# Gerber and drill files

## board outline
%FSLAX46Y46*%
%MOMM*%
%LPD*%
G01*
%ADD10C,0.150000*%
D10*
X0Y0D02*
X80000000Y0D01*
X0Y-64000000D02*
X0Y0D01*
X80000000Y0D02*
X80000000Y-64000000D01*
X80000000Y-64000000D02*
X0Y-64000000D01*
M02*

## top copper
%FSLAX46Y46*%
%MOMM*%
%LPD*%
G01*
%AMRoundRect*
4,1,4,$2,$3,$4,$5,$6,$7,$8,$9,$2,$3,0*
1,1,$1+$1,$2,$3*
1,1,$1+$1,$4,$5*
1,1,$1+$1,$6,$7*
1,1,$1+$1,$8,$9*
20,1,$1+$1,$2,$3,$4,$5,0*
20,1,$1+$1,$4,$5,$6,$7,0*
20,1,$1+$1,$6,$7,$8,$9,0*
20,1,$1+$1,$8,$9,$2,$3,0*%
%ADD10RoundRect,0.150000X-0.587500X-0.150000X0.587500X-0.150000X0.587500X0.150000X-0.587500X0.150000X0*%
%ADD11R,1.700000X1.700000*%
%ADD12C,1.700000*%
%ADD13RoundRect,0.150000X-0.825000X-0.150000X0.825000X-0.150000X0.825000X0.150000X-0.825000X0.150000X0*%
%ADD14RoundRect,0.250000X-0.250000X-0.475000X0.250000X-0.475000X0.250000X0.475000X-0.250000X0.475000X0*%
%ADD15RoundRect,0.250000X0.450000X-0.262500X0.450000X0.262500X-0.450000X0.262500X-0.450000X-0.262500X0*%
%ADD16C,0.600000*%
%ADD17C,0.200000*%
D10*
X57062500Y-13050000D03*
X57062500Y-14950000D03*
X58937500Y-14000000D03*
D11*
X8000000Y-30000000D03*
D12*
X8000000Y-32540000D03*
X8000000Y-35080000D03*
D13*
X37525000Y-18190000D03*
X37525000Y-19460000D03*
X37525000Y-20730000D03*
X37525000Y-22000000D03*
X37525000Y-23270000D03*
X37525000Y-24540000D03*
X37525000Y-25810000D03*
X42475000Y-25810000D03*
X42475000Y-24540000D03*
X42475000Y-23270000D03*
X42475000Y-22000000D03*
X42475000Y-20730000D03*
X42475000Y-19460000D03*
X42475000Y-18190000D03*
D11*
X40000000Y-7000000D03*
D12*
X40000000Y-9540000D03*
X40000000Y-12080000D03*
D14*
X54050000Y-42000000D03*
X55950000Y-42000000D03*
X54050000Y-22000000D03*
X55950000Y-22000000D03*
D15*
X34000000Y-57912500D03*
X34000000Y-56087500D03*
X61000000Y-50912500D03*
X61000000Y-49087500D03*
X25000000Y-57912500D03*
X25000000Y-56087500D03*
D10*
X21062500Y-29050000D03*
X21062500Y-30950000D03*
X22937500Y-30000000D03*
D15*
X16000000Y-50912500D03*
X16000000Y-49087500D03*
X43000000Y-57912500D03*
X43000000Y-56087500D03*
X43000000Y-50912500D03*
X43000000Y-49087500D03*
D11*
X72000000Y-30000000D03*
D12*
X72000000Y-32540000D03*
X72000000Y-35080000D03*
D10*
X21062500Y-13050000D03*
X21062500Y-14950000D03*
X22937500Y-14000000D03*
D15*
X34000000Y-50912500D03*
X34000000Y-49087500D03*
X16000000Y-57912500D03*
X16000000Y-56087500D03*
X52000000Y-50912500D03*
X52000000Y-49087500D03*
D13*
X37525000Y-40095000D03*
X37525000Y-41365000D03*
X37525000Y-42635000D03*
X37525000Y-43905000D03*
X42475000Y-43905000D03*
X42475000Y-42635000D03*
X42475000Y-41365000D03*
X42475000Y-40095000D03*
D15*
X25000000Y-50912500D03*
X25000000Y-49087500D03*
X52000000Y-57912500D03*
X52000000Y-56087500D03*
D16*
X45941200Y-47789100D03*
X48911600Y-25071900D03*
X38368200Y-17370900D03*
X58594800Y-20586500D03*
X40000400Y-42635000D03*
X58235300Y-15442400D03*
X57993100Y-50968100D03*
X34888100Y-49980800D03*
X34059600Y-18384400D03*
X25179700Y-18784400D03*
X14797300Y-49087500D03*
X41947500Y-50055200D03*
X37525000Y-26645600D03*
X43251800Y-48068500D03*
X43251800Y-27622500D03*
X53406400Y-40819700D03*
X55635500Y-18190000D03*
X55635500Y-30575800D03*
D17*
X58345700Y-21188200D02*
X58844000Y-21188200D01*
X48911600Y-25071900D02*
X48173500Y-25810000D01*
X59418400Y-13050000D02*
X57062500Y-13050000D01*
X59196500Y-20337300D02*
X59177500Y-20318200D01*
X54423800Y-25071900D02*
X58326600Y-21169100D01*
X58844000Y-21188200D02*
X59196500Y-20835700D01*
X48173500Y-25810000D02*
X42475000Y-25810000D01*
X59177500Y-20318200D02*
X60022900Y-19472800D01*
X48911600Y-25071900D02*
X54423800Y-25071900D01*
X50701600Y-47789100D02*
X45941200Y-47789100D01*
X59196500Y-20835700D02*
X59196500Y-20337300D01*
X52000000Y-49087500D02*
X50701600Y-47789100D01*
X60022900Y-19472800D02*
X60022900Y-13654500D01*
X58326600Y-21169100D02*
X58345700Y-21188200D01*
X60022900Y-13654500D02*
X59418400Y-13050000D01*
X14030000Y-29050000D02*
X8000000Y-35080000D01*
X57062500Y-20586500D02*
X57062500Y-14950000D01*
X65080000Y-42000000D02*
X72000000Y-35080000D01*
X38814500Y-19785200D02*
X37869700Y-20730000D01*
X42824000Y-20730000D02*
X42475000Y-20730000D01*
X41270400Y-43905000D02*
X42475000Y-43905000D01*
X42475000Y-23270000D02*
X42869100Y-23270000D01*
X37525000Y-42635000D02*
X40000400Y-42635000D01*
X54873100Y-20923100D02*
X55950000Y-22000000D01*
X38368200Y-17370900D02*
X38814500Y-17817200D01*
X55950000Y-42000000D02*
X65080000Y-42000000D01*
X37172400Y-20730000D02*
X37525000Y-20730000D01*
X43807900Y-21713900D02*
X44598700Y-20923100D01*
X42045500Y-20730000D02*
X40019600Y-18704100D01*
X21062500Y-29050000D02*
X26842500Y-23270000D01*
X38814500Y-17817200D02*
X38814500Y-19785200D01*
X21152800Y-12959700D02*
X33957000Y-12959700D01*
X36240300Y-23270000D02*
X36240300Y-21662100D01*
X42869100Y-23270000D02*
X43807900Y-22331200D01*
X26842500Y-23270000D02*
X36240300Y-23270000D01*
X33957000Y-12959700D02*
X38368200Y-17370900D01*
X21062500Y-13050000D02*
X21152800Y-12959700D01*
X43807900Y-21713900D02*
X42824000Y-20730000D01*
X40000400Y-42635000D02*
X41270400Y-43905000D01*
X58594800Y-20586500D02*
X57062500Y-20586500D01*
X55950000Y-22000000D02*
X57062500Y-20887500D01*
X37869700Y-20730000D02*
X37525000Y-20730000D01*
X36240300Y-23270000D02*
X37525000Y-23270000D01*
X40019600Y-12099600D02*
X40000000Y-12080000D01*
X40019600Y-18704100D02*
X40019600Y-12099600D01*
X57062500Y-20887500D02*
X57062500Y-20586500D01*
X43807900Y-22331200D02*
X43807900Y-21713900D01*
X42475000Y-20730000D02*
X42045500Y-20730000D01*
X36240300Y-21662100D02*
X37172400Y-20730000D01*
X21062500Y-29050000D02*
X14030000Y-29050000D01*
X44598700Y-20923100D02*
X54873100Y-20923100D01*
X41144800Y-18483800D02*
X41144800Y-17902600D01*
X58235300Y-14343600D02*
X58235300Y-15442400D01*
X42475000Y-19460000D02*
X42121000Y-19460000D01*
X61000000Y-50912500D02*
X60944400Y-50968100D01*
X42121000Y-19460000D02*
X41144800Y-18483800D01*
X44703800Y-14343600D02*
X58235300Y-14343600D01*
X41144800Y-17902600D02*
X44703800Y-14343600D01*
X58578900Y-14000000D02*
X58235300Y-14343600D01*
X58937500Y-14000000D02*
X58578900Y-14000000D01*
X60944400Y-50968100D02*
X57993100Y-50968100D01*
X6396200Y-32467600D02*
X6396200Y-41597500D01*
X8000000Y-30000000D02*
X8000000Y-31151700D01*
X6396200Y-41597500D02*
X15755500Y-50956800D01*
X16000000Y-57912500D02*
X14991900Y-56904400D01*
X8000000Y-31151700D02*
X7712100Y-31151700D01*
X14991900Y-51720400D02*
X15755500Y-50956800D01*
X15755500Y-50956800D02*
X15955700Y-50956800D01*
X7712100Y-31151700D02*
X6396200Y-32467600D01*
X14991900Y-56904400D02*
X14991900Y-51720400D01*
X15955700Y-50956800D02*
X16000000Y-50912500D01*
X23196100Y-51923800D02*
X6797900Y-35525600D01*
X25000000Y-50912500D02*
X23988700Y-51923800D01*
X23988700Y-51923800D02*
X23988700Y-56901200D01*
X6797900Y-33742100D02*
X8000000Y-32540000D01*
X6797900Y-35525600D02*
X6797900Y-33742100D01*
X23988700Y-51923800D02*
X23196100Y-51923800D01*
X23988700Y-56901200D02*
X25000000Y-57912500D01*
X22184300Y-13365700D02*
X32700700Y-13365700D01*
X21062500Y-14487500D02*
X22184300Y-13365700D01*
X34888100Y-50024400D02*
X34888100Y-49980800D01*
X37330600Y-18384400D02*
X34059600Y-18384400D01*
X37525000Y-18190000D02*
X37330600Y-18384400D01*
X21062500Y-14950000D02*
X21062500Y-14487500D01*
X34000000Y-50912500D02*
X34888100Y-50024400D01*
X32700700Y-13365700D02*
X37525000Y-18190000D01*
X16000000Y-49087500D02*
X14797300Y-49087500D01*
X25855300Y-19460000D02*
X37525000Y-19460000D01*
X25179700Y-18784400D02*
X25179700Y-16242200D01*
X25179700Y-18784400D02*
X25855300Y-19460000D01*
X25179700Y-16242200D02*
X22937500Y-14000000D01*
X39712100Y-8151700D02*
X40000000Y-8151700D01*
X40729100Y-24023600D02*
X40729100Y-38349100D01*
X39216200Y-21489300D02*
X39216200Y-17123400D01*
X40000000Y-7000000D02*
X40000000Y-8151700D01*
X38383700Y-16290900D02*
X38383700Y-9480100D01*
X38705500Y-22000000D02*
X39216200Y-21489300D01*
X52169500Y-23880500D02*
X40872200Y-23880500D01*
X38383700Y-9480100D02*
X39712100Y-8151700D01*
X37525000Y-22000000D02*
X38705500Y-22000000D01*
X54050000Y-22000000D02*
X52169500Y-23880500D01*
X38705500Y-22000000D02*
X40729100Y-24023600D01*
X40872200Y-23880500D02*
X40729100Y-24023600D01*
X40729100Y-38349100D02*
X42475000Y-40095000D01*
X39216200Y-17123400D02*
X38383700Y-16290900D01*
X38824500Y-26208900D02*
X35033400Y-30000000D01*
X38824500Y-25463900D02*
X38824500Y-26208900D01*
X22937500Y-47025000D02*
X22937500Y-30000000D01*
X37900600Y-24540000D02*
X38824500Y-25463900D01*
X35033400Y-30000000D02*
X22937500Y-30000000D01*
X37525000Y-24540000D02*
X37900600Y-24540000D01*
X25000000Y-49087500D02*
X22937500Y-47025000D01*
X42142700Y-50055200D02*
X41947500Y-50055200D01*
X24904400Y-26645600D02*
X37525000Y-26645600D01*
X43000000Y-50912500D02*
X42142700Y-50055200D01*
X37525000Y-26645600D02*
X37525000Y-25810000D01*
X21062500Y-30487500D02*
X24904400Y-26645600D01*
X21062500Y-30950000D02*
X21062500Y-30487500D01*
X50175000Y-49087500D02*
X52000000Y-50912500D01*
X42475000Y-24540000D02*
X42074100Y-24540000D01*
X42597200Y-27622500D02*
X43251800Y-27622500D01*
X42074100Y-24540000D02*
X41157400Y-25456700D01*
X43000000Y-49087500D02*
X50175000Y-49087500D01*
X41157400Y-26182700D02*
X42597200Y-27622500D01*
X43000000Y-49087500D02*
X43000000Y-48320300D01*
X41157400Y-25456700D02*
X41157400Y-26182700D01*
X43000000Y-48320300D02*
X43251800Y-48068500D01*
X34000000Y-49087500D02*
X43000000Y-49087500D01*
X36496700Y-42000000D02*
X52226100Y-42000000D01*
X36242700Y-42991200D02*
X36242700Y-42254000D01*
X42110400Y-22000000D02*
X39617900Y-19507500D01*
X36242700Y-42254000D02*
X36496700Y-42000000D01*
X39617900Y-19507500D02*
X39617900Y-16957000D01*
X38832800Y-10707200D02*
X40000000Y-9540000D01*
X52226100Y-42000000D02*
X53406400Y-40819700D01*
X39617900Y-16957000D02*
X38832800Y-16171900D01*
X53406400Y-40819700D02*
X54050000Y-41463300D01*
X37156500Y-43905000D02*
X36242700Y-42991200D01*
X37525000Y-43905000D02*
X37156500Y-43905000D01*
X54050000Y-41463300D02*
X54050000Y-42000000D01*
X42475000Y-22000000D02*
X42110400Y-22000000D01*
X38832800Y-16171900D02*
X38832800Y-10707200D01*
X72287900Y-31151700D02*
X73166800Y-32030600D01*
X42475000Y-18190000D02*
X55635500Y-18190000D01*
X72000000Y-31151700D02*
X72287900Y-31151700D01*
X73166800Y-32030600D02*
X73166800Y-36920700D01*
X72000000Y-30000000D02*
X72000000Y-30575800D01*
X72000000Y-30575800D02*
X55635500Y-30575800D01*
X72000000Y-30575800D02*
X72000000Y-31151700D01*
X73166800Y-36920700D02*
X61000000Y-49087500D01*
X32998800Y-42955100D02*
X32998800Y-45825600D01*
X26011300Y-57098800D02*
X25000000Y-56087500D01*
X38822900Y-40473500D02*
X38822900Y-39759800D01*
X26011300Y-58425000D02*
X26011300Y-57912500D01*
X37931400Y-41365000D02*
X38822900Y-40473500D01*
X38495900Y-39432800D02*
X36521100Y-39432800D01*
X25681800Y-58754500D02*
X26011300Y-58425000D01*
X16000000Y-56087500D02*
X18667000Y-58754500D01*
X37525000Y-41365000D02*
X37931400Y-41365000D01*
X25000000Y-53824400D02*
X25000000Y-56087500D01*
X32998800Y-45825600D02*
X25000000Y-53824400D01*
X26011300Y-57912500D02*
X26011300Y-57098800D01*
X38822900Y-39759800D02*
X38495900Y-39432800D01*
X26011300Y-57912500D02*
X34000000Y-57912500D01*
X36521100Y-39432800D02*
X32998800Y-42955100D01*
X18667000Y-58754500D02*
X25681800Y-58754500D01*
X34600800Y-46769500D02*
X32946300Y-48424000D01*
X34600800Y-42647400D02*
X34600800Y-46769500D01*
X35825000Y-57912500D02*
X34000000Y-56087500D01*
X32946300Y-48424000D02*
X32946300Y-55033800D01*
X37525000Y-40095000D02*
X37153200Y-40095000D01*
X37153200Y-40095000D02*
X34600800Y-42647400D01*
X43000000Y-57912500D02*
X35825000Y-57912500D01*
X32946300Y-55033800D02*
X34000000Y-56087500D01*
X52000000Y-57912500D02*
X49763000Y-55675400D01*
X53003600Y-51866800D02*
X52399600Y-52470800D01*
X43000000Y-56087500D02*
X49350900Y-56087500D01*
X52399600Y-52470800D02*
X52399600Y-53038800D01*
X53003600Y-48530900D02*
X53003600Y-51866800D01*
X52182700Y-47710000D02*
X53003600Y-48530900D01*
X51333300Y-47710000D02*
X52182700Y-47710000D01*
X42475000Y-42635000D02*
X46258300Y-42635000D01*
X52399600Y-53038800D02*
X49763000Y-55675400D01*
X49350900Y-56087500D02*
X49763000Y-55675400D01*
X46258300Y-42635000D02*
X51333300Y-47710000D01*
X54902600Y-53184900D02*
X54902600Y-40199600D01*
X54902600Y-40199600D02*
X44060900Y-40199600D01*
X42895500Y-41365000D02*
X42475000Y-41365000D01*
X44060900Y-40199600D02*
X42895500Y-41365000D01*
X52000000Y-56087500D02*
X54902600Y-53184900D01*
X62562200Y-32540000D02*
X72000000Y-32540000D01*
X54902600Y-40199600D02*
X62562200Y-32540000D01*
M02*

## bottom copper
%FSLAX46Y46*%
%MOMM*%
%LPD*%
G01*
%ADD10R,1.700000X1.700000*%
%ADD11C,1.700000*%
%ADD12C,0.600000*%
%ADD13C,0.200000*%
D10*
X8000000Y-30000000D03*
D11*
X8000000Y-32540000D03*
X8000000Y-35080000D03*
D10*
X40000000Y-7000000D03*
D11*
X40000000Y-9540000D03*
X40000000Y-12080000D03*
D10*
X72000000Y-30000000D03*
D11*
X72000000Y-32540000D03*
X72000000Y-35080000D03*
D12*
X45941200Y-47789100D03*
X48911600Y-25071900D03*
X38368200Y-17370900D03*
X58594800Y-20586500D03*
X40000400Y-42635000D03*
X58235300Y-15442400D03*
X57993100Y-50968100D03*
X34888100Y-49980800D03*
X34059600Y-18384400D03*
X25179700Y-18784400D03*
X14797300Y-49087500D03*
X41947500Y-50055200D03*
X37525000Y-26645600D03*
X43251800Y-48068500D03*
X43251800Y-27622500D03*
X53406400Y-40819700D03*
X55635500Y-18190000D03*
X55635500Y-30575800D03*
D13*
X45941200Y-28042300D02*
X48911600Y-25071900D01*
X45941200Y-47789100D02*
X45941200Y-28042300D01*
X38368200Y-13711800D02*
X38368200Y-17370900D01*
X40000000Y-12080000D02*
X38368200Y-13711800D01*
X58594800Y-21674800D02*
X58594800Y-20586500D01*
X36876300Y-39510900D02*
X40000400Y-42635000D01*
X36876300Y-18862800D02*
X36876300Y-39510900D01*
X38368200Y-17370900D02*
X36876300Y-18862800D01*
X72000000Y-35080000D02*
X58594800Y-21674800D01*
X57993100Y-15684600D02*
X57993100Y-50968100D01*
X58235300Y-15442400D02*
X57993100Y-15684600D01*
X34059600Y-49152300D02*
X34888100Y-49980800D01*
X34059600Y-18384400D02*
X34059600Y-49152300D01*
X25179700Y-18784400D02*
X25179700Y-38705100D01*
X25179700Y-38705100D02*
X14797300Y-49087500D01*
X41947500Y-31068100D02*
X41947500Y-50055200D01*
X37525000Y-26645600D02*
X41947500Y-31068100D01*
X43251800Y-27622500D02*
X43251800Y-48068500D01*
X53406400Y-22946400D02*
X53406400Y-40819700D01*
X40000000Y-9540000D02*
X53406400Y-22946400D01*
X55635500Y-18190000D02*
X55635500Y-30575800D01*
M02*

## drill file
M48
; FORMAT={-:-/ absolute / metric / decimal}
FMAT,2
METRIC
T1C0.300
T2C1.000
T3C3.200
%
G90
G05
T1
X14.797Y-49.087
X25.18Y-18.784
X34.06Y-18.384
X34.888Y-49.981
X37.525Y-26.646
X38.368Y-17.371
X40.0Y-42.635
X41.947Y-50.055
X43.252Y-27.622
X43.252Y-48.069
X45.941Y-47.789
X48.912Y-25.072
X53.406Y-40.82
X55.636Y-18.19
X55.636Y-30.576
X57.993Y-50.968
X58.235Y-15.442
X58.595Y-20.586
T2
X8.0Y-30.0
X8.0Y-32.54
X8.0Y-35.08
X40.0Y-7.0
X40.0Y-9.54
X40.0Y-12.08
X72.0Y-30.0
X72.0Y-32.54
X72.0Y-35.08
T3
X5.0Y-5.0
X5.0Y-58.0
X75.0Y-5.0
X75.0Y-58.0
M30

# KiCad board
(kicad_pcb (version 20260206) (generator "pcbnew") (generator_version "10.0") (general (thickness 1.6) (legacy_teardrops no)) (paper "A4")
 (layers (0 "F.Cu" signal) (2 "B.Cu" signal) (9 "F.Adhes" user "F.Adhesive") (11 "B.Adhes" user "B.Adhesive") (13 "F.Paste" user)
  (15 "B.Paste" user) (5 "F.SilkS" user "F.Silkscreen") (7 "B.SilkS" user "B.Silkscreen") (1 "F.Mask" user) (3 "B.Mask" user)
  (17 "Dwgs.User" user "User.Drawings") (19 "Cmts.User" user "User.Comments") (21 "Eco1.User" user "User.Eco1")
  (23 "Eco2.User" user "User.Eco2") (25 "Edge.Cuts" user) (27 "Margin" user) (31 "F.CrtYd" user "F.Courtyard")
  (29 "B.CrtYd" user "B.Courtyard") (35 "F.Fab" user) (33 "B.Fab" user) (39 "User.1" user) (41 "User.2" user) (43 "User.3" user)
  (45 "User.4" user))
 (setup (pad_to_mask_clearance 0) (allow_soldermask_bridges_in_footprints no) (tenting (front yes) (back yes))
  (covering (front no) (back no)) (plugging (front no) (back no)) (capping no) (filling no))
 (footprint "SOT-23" (layer "F.Cu") (at 58 14)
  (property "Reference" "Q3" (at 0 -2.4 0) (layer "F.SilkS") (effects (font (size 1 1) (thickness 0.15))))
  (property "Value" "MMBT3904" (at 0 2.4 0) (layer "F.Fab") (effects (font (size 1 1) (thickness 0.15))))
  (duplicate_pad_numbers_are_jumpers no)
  (pad "1" smd roundrect (at -0.9375 -0.95) (size 1.475 0.6) (layers "F.Cu" "F.Mask" "F.Paste") (roundrect_rratio 0.25) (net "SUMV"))
  (pad "2" smd roundrect (at -0.9375 0.95) (size 1.475 0.6) (layers "F.Cu" "F.Mask" "F.Paste") (roundrect_rratio 0.25) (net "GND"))
  (pad "3" smd roundrect (at 0.9375 0) (size 1.475 0.6) (layers "F.Cu" "F.Mask" "F.Paste") (roundrect_rratio 0.25) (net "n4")))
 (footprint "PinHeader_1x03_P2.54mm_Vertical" (layer "F.Cu") (at 8 30)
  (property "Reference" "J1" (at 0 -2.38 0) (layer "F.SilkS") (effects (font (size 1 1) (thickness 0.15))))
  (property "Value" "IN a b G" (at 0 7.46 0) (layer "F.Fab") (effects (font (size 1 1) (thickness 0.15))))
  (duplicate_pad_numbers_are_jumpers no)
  (pad "1" thru_hole rect (at 0 0) (size 1.7 1.7) (drill 1) (layers "*.Cu" "*.Mask") (remove_unused_layers no) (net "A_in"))
  (pad "2" thru_hole circle (at 0 2.54) (size 1.7 1.7) (drill 1) (layers "*.Cu" "*.Mask") (remove_unused_layers no) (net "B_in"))
  (pad "3" thru_hole circle (at 0 5.08) (size 1.7 1.7) (drill 1) (layers "*.Cu" "*.Mask") (remove_unused_layers no) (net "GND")))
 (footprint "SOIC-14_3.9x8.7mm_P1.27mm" (layer "F.Cu") (at 40 22)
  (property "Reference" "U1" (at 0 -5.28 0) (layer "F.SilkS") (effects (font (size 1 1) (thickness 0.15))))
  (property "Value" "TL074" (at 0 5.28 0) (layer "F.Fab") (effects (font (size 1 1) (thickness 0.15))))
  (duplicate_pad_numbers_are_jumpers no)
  (pad "1" smd roundrect (at -2.475 -3.81) (size 1.95 0.6) (layers "F.Cu" "F.Mask" "F.Paste") (roundrect_rratio 0.25) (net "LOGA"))
  (pad "2" smd roundrect (at -2.475 -2.54) (size 1.95 0.6) (layers "F.Cu" "F.Mask" "F.Paste") (roundrect_rratio 0.25) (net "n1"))
  (pad "3" smd roundrect (at -2.475 -1.27) (size 1.95 0.6) (layers "F.Cu" "F.Mask" "F.Paste") (roundrect_rratio 0.25) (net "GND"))
  (pad "4" smd roundrect (at -2.475 0) (size 1.95 0.6) (layers "F.Cu" "F.Mask" "F.Paste") (roundrect_rratio 0.25) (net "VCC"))
  (pad "5" smd roundrect (at -2.475 1.27) (size 1.95 0.6) (layers "F.Cu" "F.Mask" "F.Paste") (roundrect_rratio 0.25) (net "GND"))
  (pad "6" smd roundrect (at -2.475 2.54) (size 1.95 0.6) (layers "F.Cu" "F.Mask" "F.Paste") (roundrect_rratio 0.25) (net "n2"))
  (pad "7" smd roundrect (at -2.475 3.81) (size 1.95 0.6) (layers "F.Cu" "F.Mask" "F.Paste") (roundrect_rratio 0.25) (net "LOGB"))
  (pad "8" smd roundrect (at 2.475 3.81) (size 1.95 0.6) (layers "F.Cu" "F.Mask" "F.Paste") (roundrect_rratio 0.25) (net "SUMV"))
  (pad "9" smd roundrect (at 2.475 2.54) (size 1.95 0.6) (layers "F.Cu" "F.Mask" "F.Paste") (roundrect_rratio 0.25) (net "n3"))
  (pad "10" smd roundrect (at 2.475 1.27) (size 1.95 0.6) (layers "F.Cu" "F.Mask" "F.Paste") (roundrect_rratio 0.25) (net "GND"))
  (pad "11" smd roundrect (at 2.475 0) (size 1.95 0.6) (layers "F.Cu" "F.Mask" "F.Paste") (roundrect_rratio 0.25) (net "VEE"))
  (pad "12" smd roundrect (at 2.475 -1.27) (size 1.95 0.6) (layers "F.Cu" "F.Mask" "F.Paste") (roundrect_rratio 0.25) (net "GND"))
  (pad "13" smd roundrect (at 2.475 -2.54) (size 1.95 0.6) (layers "F.Cu" "F.Mask" "F.Paste") (roundrect_rratio 0.25) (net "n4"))
  (pad "14" smd roundrect (at 2.475 -3.81) (size 1.95 0.6) (layers "F.Cu" "F.Mask" "F.Paste") (roundrect_rratio 0.25) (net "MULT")))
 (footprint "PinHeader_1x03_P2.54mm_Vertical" (layer "F.Cu") (at 40 7)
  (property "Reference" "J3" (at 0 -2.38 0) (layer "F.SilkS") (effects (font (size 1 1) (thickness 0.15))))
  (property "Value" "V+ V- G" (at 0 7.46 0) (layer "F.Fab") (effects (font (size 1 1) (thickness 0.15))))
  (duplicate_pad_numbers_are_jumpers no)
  (pad "1" thru_hole rect (at 0 0) (size 1.7 1.7) (drill 1) (layers "*.Cu" "*.Mask") (remove_unused_layers no) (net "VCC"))
  (pad "2" thru_hole circle (at 0 2.54) (size 1.7 1.7) (drill 1) (layers "*.Cu" "*.Mask") (remove_unused_layers no) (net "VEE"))
  (pad "3" thru_hole circle (at 0 5.08) (size 1.7 1.7) (drill 1) (layers "*.Cu" "*.Mask") (remove_unused_layers no) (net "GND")))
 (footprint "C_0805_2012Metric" (layer "F.Cu") (at 55 42)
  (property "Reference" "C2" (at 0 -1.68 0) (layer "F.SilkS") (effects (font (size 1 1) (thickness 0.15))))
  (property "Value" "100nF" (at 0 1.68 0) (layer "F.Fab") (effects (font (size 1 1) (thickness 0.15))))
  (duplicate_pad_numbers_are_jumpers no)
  (pad "1" smd roundrect (at -0.95 0) (size 1 1.45) (layers "F.Cu" "F.Mask" "F.Paste") (roundrect_rratio 0.25) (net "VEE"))
  (pad "2" smd roundrect (at 0.95 0) (size 1 1.45) (layers "F.Cu" "F.Mask" "F.Paste") (roundrect_rratio 0.25) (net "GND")))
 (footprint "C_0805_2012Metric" (layer "F.Cu") (at 55 22)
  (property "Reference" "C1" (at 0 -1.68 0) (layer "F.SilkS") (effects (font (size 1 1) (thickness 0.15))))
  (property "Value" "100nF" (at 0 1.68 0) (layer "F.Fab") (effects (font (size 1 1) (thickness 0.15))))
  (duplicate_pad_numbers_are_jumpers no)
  (pad "1" smd roundrect (at -0.95 0) (size 1 1.45) (layers "F.Cu" "F.Mask" "F.Paste") (roundrect_rratio 0.25) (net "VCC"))
  (pad "2" smd roundrect (at 0.95 0) (size 1 1.45) (layers "F.Cu" "F.Mask" "F.Paste") (roundrect_rratio 0.25) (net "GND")))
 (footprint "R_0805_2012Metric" (layer "F.Cu") (at 34 57 90)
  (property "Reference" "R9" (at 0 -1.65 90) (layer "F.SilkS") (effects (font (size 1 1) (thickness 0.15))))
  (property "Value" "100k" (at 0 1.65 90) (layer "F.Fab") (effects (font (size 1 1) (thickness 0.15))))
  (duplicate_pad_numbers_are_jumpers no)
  (pad "1" smd roundrect (at -0.9125 0 90) (size 1.025 1.4) (layers "F.Cu" "F.Mask" "F.Paste") (roundrect_rratio 0.243902) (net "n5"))
  (pad "2" smd roundrect (at 0.9125 0 90) (size 1.025 1.4) (layers "F.Cu" "F.Mask" "F.Paste") (roundrect_rratio 0.243902) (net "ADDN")))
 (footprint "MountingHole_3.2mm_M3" (layer "F.Cu") (at 5 58)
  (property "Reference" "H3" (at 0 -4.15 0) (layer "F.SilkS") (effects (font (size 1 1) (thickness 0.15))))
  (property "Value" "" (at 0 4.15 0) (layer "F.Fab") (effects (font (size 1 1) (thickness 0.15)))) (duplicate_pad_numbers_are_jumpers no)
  (pad "" np_thru_hole circle (at 0 0) (size 3.2 3.2) (drill 3.2) (layers "*.Cu" "*.Mask")))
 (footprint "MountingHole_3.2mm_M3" (layer "F.Cu") (at 75 5)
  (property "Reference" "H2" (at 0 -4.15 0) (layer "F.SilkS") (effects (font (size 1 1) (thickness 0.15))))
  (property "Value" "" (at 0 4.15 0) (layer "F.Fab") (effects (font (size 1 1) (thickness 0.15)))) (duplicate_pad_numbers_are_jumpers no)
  (pad "" np_thru_hole circle (at 0 0) (size 3.2 3.2) (drill 3.2) (layers "*.Cu" "*.Mask")))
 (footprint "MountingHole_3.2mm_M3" (layer "F.Cu") (at 5 5)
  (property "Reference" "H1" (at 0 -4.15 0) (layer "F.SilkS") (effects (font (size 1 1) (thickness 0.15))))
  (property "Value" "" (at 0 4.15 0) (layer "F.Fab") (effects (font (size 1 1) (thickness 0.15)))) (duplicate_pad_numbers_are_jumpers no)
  (pad "" np_thru_hole circle (at 0 0) (size 3.2 3.2) (drill 3.2) (layers "*.Cu" "*.Mask")))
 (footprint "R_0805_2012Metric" (layer "F.Cu") (at 61 50 90)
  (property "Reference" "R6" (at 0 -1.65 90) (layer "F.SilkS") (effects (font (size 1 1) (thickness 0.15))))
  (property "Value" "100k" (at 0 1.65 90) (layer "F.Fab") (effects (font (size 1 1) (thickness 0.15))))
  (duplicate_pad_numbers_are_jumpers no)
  (pad "1" smd roundrect (at -0.9125 0 90) (size 1.025 1.4) (layers "F.Cu" "F.Mask" "F.Paste") (roundrect_rratio 0.243902) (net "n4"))
  (pad "2" smd roundrect (at 0.9125 0 90) (size 1.025 1.4) (layers "F.Cu" "F.Mask" "F.Paste") (roundrect_rratio 0.243902) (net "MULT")))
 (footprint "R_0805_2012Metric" (layer "F.Cu") (at 25 57 90)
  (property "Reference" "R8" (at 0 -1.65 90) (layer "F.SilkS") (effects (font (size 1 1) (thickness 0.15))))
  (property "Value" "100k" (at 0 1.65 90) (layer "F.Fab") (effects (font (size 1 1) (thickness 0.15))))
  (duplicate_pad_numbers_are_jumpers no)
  (pad "1" smd roundrect (at -0.9125 0 90) (size 1.025 1.4) (layers "F.Cu" "F.Mask" "F.Paste") (roundrect_rratio 0.243902) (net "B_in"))
  (pad "2" smd roundrect (at 0.9125 0 90) (size 1.025 1.4) (layers "F.Cu" "F.Mask" "F.Paste") (roundrect_rratio 0.243902) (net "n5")))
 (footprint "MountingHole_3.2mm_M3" (layer "F.Cu") (at 75 58)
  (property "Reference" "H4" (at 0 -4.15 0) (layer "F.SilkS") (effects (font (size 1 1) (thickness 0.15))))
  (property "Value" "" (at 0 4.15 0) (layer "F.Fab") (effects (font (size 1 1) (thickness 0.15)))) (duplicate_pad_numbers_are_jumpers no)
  (pad "" np_thru_hole circle (at 0 0) (size 3.2 3.2) (drill 3.2) (layers "*.Cu" "*.Mask")))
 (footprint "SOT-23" (layer "F.Cu") (at 22 30)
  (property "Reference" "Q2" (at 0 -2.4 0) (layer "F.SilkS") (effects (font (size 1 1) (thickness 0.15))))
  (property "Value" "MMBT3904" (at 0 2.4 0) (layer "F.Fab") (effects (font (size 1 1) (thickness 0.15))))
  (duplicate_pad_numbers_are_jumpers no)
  (pad "1" smd roundrect (at -0.9375 -0.95) (size 1.475 0.6) (layers "F.Cu" "F.Mask" "F.Paste") (roundrect_rratio 0.25) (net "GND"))
  (pad "2" smd roundrect (at -0.9375 0.95) (size 1.475 0.6) (layers "F.Cu" "F.Mask" "F.Paste") (roundrect_rratio 0.25) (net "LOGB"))
  (pad "3" smd roundrect (at 0.9375 0) (size 1.475 0.6) (layers "F.Cu" "F.Mask" "F.Paste") (roundrect_rratio 0.25) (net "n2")))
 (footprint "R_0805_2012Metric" (layer "F.Cu") (at 16 50 90)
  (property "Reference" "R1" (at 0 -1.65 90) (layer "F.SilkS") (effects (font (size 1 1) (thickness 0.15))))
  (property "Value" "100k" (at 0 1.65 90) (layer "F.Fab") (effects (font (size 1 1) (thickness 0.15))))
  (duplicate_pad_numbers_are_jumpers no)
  (pad "1" smd roundrect (at -0.9125 0 90) (size 1.025 1.4) (layers "F.Cu" "F.Mask" "F.Paste") (roundrect_rratio 0.243902) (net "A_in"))
  (pad "2" smd roundrect (at 0.9125 0 90) (size 1.025 1.4) (layers "F.Cu" "F.Mask" "F.Paste") (roundrect_rratio 0.243902) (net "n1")))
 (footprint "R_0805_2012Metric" (layer "F.Cu") (at 43 57 90)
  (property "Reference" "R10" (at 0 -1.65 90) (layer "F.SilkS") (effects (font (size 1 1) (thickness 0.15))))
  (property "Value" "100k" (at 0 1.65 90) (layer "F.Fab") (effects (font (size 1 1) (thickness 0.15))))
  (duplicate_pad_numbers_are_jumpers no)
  (pad "1" smd roundrect (at -0.9125 0 90) (size 1.025 1.4) (layers "F.Cu" "F.Mask" "F.Paste") (roundrect_rratio 0.243902) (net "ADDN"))
  (pad "2" smd roundrect (at 0.9125 0 90) (size 1.025 1.4) (layers "F.Cu" "F.Mask" "F.Paste") (roundrect_rratio 0.243902) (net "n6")))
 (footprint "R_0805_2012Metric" (layer "F.Cu") (at 43 50 90)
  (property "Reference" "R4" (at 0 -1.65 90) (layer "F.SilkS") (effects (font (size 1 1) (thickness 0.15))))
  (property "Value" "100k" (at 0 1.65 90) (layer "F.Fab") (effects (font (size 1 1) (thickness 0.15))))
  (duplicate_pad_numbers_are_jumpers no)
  (pad "1" smd roundrect (at -0.9125 0 90) (size 1.025 1.4) (layers "F.Cu" "F.Mask" "F.Paste") (roundrect_rratio 0.243902) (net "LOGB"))
  (pad "2" smd roundrect (at 0.9125 0 90) (size 1.025 1.4) (layers "F.Cu" "F.Mask" "F.Paste") (roundrect_rratio 0.243902) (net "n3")))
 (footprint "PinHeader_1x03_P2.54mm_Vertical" (layer "F.Cu") (at 72 30)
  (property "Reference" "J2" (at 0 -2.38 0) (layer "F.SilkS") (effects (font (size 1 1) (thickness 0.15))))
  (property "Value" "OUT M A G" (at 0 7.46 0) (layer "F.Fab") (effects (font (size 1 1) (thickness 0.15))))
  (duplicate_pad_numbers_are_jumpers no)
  (pad "1" thru_hole rect (at 0 0) (size 1.7 1.7) (drill 1) (layers "*.Cu" "*.Mask") (remove_unused_layers no) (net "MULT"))
  (pad "2" thru_hole circle (at 0 2.54) (size 1.7 1.7) (drill 1) (layers "*.Cu" "*.Mask") (remove_unused_layers no) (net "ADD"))
  (pad "3" thru_hole circle (at 0 5.08) (size 1.7 1.7) (drill 1) (layers "*.Cu" "*.Mask") (remove_unused_layers no) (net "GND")))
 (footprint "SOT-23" (layer "F.Cu") (at 22 14)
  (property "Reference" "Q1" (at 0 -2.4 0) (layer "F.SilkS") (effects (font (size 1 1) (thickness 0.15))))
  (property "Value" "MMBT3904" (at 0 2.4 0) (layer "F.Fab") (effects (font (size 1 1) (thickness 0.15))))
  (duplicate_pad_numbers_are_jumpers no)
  (pad "1" smd roundrect (at -0.9375 -0.95) (size 1.475 0.6) (layers "F.Cu" "F.Mask" "F.Paste") (roundrect_rratio 0.25) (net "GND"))
  (pad "2" smd roundrect (at -0.9375 0.95) (size 1.475 0.6) (layers "F.Cu" "F.Mask" "F.Paste") (roundrect_rratio 0.25) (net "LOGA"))
  (pad "3" smd roundrect (at 0.9375 0) (size 1.475 0.6) (layers "F.Cu" "F.Mask" "F.Paste") (roundrect_rratio 0.25) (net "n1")))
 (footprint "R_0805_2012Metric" (layer "F.Cu") (at 34 50 90)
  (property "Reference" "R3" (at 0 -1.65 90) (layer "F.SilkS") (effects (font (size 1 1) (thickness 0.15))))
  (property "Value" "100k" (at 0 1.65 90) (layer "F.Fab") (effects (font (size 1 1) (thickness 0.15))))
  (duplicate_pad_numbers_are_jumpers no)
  (pad "1" smd roundrect (at -0.9125 0 90) (size 1.025 1.4) (layers "F.Cu" "F.Mask" "F.Paste") (roundrect_rratio 0.243902) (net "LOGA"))
  (pad "2" smd roundrect (at 0.9125 0 90) (size 1.025 1.4) (layers "F.Cu" "F.Mask" "F.Paste") (roundrect_rratio 0.243902) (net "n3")))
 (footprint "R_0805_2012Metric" (layer "F.Cu") (at 16 57 90)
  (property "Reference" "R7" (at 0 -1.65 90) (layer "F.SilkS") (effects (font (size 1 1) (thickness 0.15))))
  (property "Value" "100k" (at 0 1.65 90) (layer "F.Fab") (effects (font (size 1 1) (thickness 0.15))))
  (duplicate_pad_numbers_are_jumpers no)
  (pad "1" smd roundrect (at -0.9125 0 90) (size 1.025 1.4) (layers "F.Cu" "F.Mask" "F.Paste") (roundrect_rratio 0.243902) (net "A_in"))
  (pad "2" smd roundrect (at 0.9125 0 90) (size 1.025 1.4) (layers "F.Cu" "F.Mask" "F.Paste") (roundrect_rratio 0.243902) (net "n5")))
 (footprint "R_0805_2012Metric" (layer "F.Cu") (at 52 50 90)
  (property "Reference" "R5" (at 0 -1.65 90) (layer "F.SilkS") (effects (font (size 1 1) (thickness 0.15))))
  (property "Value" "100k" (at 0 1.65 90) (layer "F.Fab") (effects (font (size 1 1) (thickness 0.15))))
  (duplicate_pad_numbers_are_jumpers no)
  (pad "1" smd roundrect (at -0.9125 0 90) (size 1.025 1.4) (layers "F.Cu" "F.Mask" "F.Paste") (roundrect_rratio 0.243902) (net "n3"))
  (pad "2" smd roundrect (at 0.9125 0 90) (size 1.025 1.4) (layers "F.Cu" "F.Mask" "F.Paste") (roundrect_rratio 0.243902) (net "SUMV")))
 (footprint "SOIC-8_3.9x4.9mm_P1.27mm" (layer "F.Cu") (at 40 42)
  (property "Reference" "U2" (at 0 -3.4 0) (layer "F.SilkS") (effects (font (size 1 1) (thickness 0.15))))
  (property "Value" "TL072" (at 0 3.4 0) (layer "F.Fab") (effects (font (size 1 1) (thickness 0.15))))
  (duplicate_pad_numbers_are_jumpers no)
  (pad "1" smd roundrect (at -2.475 -1.905) (size 1.95 0.6) (layers "F.Cu" "F.Mask" "F.Paste") (roundrect_rratio 0.25) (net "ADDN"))
  (pad "2" smd roundrect (at -2.475 -0.635) (size 1.95 0.6) (layers "F.Cu" "F.Mask" "F.Paste") (roundrect_rratio 0.25) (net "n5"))
  (pad "3" smd roundrect (at -2.475 0.635) (size 1.95 0.6) (layers "F.Cu" "F.Mask" "F.Paste") (roundrect_rratio 0.25) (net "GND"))
  (pad "4" smd roundrect (at -2.475 1.905) (size 1.95 0.6) (layers "F.Cu" "F.Mask" "F.Paste") (roundrect_rratio 0.25) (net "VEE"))
  (pad "5" smd roundrect (at 2.475 1.905) (size 1.95 0.6) (layers "F.Cu" "F.Mask" "F.Paste") (roundrect_rratio 0.25) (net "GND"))
  (pad "6" smd roundrect (at 2.475 0.635) (size 1.95 0.6) (layers "F.Cu" "F.Mask" "F.Paste") (roundrect_rratio 0.25) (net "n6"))
  (pad "7" smd roundrect (at 2.475 -0.635) (size 1.95 0.6) (layers "F.Cu" "F.Mask" "F.Paste") (roundrect_rratio 0.25) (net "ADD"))
  (pad "8" smd roundrect (at 2.475 -1.905) (size 1.95 0.6) (layers "F.Cu" "F.Mask" "F.Paste") (roundrect_rratio 0.25) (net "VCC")))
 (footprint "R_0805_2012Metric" (layer "F.Cu") (at 25 50 90)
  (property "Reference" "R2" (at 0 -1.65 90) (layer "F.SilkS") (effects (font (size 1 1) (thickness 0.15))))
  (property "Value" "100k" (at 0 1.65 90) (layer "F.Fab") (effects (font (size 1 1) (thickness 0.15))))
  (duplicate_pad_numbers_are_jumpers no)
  (pad "1" smd roundrect (at -0.9125 0 90) (size 1.025 1.4) (layers "F.Cu" "F.Mask" "F.Paste") (roundrect_rratio 0.243902) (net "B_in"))
  (pad "2" smd roundrect (at 0.9125 0 90) (size 1.025 1.4) (layers "F.Cu" "F.Mask" "F.Paste") (roundrect_rratio 0.243902) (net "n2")))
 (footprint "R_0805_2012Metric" (layer "F.Cu") (at 52 57 90)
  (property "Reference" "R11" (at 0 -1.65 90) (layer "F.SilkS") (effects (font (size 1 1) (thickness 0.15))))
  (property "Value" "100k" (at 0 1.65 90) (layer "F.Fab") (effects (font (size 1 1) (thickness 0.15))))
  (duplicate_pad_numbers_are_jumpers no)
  (pad "1" smd roundrect (at -0.9125 0 90) (size 1.025 1.4) (layers "F.Cu" "F.Mask" "F.Paste") (roundrect_rratio 0.243902) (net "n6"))
  (pad "2" smd roundrect (at 0.9125 0 90) (size 1.025 1.4) (layers "F.Cu" "F.Mask" "F.Paste") (roundrect_rratio 0.243902) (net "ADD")))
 (gr_line (start 0 0) (end 80 0) (stroke (width 0.15) (type default)) (layer "Edge.Cuts"))
 (gr_line (start 0 64) (end 0 0) (stroke (width 0.15) (type default)) (layer "Edge.Cuts"))
 (gr_line (start 80 0) (end 80 64) (stroke (width 0.15) (type default)) (layer "Edge.Cuts"))
 (gr_line (start 80 64) (end 0 64) (stroke (width 0.15) (type default)) (layer "Edge.Cuts"))
 (segment (start 58.3457 21.1882) (end 58.844 21.1882) (width 0.2) (layer "F.Cu") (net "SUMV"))
 (segment (start 48.9116 25.0719) (end 48.1735 25.81) (width 0.2) (layer "F.Cu") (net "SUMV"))
 (segment (start 59.4184 13.05) (end 57.0625 13.05) (width 0.2) (layer "F.Cu") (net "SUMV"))
 (segment (start 59.1965 20.3373) (end 59.1775 20.3182) (width 0.2) (layer "F.Cu") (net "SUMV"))
 (segment (start 54.4238 25.0719) (end 58.3266 21.1691) (width 0.2) (layer "F.Cu") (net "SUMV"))
 (segment (start 58.844 21.1882) (end 59.1965 20.8357) (width 0.2) (layer "F.Cu") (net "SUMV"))
 (segment (start 48.1735 25.81) (end 42.475 25.81) (width 0.2) (layer "F.Cu") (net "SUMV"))
 (segment (start 59.1775 20.3182) (end 60.0229 19.4728) (width 0.2) (layer "F.Cu") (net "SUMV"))
 (segment (start 48.9116 25.0719) (end 54.4238 25.0719) (width 0.2) (layer "F.Cu") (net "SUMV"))
 (segment (start 50.7016 47.7891) (end 45.9412 47.7891) (width 0.2) (layer "F.Cu") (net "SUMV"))
 (segment (start 59.1965 20.8357) (end 59.1965 20.3373) (width 0.2) (layer "F.Cu") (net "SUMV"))
 (segment (start 52 49.0875) (end 50.7016 47.7891) (width 0.2) (layer "F.Cu") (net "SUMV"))
 (segment (start 60.0229 19.4728) (end 60.0229 13.6545) (width 0.2) (layer "F.Cu") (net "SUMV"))
 (segment (start 58.3266 21.1691) (end 58.3457 21.1882) (width 0.2) (layer "F.Cu") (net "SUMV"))
 (segment (start 60.0229 13.6545) (end 59.4184 13.05) (width 0.2) (layer "F.Cu") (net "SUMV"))
 (via (at 45.9412 47.7891) (size 0.6) (drill 0.3) (layers "F.Cu" "B.Cu") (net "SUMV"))
 (via (at 48.9116 25.0719) (size 0.6) (drill 0.3) (layers "F.Cu" "B.Cu") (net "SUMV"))
 (segment (start 45.9412 28.0423) (end 48.9116 25.0719) (width 0.2) (layer "B.Cu") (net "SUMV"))
 (segment (start 45.9412 47.7891) (end 45.9412 28.0423) (width 0.2) (layer "B.Cu") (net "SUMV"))
 (segment (start 14.03 29.05) (end 8 35.08) (width 0.2) (layer "F.Cu") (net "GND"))
 (segment (start 57.0625 20.5865) (end 57.0625 14.95) (width 0.2) (layer "F.Cu") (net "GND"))
 (segment (start 65.08 42) (end 72 35.08) (width 0.2) (layer "F.Cu") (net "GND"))
 (segment (start 38.8145 19.7852) (end 37.8697 20.73) (width 0.2) (layer "F.Cu") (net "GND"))
 (segment (start 42.824 20.73) (end 42.475 20.73) (width 0.2) (layer "F.Cu") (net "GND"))
 (segment (start 41.2704 43.905) (end 42.475 43.905) (width 0.2) (layer "F.Cu") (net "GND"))
 (segment (start 42.475 23.27) (end 42.8691 23.27) (width 0.2) (layer "F.Cu") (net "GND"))
 (segment (start 37.525 42.635) (end 40.0004 42.635) (width 0.2) (layer "F.Cu") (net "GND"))
 (segment (start 54.8731 20.9231) (end 55.95 22) (width 0.2) (layer "F.Cu") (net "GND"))
 (segment (start 38.3682 17.3709) (end 38.8145 17.8172) (width 0.2) (layer "F.Cu") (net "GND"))
 (segment (start 55.95 42) (end 65.08 42) (width 0.2) (layer "F.Cu") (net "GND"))
 (segment (start 37.1724 20.73) (end 37.525 20.73) (width 0.2) (layer "F.Cu") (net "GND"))
 (segment (start 43.8079 21.7139) (end 44.5987 20.9231) (width 0.2) (layer "F.Cu") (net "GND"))
 (segment (start 42.0455 20.73) (end 40.0196 18.7041) (width 0.2) (layer "F.Cu") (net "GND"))
 (segment (start 21.0625 29.05) (end 26.8425 23.27) (width 0.2) (layer "F.Cu") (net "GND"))
 (segment (start 38.8145 17.8172) (end 38.8145 19.7852) (width 0.2) (layer "F.Cu") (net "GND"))
 (segment (start 21.1528 12.9597) (end 33.957 12.9597) (width 0.2) (layer "F.Cu") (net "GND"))
 (segment (start 36.2403 23.27) (end 36.2403 21.6621) (width 0.2) (layer "F.Cu") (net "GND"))
 (segment (start 42.8691 23.27) (end 43.8079 22.3312) (width 0.2) (layer "F.Cu") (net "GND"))
 (segment (start 26.8425 23.27) (end 36.2403 23.27) (width 0.2) (layer "F.Cu") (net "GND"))
 (segment (start 33.957 12.9597) (end 38.3682 17.3709) (width 0.2) (layer "F.Cu") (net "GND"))
 (segment (start 21.0625 13.05) (end 21.1528 12.9597) (width 0.2) (layer "F.Cu") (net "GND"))
 (segment (start 43.8079 21.7139) (end 42.824 20.73) (width 0.2) (layer "F.Cu") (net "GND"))
 (segment (start 40.0004 42.635) (end 41.2704 43.905) (width 0.2) (layer "F.Cu") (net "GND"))
 (segment (start 58.5948 20.5865) (end 57.0625 20.5865) (width 0.2) (layer "F.Cu") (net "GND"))
 (segment (start 55.95 22) (end 57.0625 20.8875) (width 0.2) (layer "F.Cu") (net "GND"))
 (segment (start 37.8697 20.73) (end 37.525 20.73) (width 0.2) (layer "F.Cu") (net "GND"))
 (segment (start 36.2403 23.27) (end 37.525 23.27) (width 0.2) (layer "F.Cu") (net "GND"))
 (segment (start 40.0196 12.0996) (end 40 12.08) (width 0.2) (layer "F.Cu") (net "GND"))
 (segment (start 40.0196 18.7041) (end 40.0196 12.0996) (width 0.2) (layer "F.Cu") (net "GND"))
 (segment (start 57.0625 20.8875) (end 57.0625 20.5865) (width 0.2) (layer "F.Cu") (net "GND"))
 (segment (start 43.8079 22.3312) (end 43.8079 21.7139) (width 0.2) (layer "F.Cu") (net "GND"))
 (segment (start 42.475 20.73) (end 42.0455 20.73) (width 0.2) (layer "F.Cu") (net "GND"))
 (segment (start 36.2403 21.6621) (end 37.1724 20.73) (width 0.2) (layer "F.Cu") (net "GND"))
 (segment (start 21.0625 29.05) (end 14.03 29.05) (width 0.2) (layer "F.Cu") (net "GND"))
 (segment (start 44.5987 20.9231) (end 54.8731 20.9231) (width 0.2) (layer "F.Cu") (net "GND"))
 (via (at 38.3682 17.3709) (size 0.6) (drill 0.3) (layers "F.Cu" "B.Cu") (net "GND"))
 (via (at 58.5948 20.5865) (size 0.6) (drill 0.3) (layers "F.Cu" "B.Cu") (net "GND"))
 (via (at 40.0004 42.635) (size 0.6) (drill 0.3) (layers "F.Cu" "B.Cu") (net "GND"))
 (segment (start 38.3682 13.7118) (end 38.3682 17.3709) (width 0.2) (layer "B.Cu") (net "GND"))
 (segment (start 40 12.08) (end 38.3682 13.7118) (width 0.2) (layer "B.Cu") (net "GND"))
 (segment (start 58.5948 21.6748) (end 58.5948 20.5865) (width 0.2) (layer "B.Cu") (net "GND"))
 (segment (start 36.8763 39.5109) (end 40.0004 42.635) (width 0.2) (layer "B.Cu") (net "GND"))
 (segment (start 36.8763 18.8628) (end 36.8763 39.5109) (width 0.2) (layer "B.Cu") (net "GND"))
 (segment (start 38.3682 17.3709) (end 36.8763 18.8628) (width 0.2) (layer "B.Cu") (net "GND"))
 (segment (start 72 35.08) (end 58.5948 21.6748) (width 0.2) (layer "B.Cu") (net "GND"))
 (segment (start 41.1448 18.4838) (end 41.1448 17.9026) (width 0.2) (layer "F.Cu") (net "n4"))
 (segment (start 58.2353 14.3436) (end 58.2353 15.4424) (width 0.2) (layer "F.Cu") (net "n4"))
 (segment (start 42.475 19.46) (end 42.121 19.46) (width 0.2) (layer "F.Cu") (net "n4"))
 (segment (start 61 50.9125) (end 60.9444 50.9681) (width 0.2) (layer "F.Cu") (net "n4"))
 (segment (start 42.121 19.46) (end 41.1448 18.4838) (width 0.2) (layer "F.Cu") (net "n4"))
 (segment (start 44.7038 14.3436) (end 58.2353 14.3436) (width 0.2) (layer "F.Cu") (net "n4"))
 (segment (start 41.1448 17.9026) (end 44.7038 14.3436) (width 0.2) (layer "F.Cu") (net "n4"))
 (segment (start 58.5789 14) (end 58.2353 14.3436) (width 0.2) (layer "F.Cu") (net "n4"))
 (segment (start 58.9375 14) (end 58.5789 14) (width 0.2) (layer "F.Cu") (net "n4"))
 (segment (start 60.9444 50.9681) (end 57.9931 50.9681) (width 0.2) (layer "F.Cu") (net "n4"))
 (via (at 58.2353 15.4424) (size 0.6) (drill 0.3) (layers "F.Cu" "B.Cu") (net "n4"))
 (via (at 57.9931 50.9681) (size 0.6) (drill 0.3) (layers "F.Cu" "B.Cu") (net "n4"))
 (segment (start 57.9931 15.6846) (end 57.9931 50.9681) (width 0.2) (layer "B.Cu") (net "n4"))
 (segment (start 58.2353 15.4424) (end 57.9931 15.6846) (width 0.2) (layer "B.Cu") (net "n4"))
 (segment (start 6.3962 32.4676) (end 6.3962 41.5975) (width 0.2) (layer "F.Cu") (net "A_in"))
 (segment (start 8 30) (end 8 31.1517) (width 0.2) (layer "F.Cu") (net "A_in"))
 (segment (start 6.3962 41.5975) (end 15.7555 50.9568) (width 0.2) (layer "F.Cu") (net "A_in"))
 (segment (start 16 57.9125) (end 14.9919 56.9044) (width 0.2) (layer "F.Cu") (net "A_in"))
 (segment (start 8 31.1517) (end 7.7121 31.1517) (width 0.2) (layer "F.Cu") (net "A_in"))
 (segment (start 14.9919 51.7204) (end 15.7555 50.9568) (width 0.2) (layer "F.Cu") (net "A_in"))
 (segment (start 15.7555 50.9568) (end 15.9557 50.9568) (width 0.2) (layer "F.Cu") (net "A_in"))
 (segment (start 7.7121 31.1517) (end 6.3962 32.4676) (width 0.2) (layer "F.Cu") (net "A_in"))
 (segment (start 14.9919 56.9044) (end 14.9919 51.7204) (width 0.2) (layer "F.Cu") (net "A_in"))
 (segment (start 15.9557 50.9568) (end 16 50.9125) (width 0.2) (layer "F.Cu") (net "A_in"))
 (segment (start 23.1961 51.9238) (end 6.7979 35.5256) (width 0.2) (layer "F.Cu") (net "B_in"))
 (segment (start 25 50.9125) (end 23.9887 51.9238) (width 0.2) (layer "F.Cu") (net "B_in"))
 (segment (start 23.9887 51.9238) (end 23.9887 56.9012) (width 0.2) (layer "F.Cu") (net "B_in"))
 (segment (start 6.7979 33.7421) (end 8 32.54) (width 0.2) (layer "F.Cu") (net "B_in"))
 (segment (start 6.7979 35.5256) (end 6.7979 33.7421) (width 0.2) (layer "F.Cu") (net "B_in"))
 (segment (start 23.9887 51.9238) (end 23.1961 51.9238) (width 0.2) (layer "F.Cu") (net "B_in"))
 (segment (start 23.9887 56.9012) (end 25 57.9125) (width 0.2) (layer "F.Cu") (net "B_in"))
 (segment (start 22.1843 13.3657) (end 32.7007 13.3657) (width 0.2) (layer "F.Cu") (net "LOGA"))
 (segment (start 21.0625 14.4875) (end 22.1843 13.3657) (width 0.2) (layer "F.Cu") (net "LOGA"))
 (segment (start 34.8881 50.0244) (end 34.8881 49.9808) (width 0.2) (layer "F.Cu") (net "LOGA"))
 (segment (start 37.3306 18.3844) (end 34.0596 18.3844) (width 0.2) (layer "F.Cu") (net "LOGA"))
 (segment (start 37.525 18.19) (end 37.3306 18.3844) (width 0.2) (layer "F.Cu") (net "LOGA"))
 (segment (start 21.0625 14.95) (end 21.0625 14.4875) (width 0.2) (layer "F.Cu") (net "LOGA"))
 (segment (start 34 50.9125) (end 34.8881 50.0244) (width 0.2) (layer "F.Cu") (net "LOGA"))
 (segment (start 32.7007 13.3657) (end 37.525 18.19) (width 0.2) (layer "F.Cu") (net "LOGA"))
 (via (at 34.8881 49.9808) (size 0.6) (drill 0.3) (layers "F.Cu" "B.Cu") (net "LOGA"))
 (via (at 34.0596 18.3844) (size 0.6) (drill 0.3) (layers "F.Cu" "B.Cu") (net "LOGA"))
 (segment (start 34.0596 49.1523) (end 34.8881 49.9808) (width 0.2) (layer "B.Cu") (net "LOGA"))
 (segment (start 34.0596 18.3844) (end 34.0596 49.1523) (width 0.2) (layer "B.Cu") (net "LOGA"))
 (segment (start 16 49.0875) (end 14.7973 49.0875) (width 0.2) (layer "F.Cu") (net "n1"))
 (segment (start 25.8553 19.46) (end 37.525 19.46) (width 0.2) (layer "F.Cu") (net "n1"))
 (segment (start 25.1797 18.7844) (end 25.1797 16.2422) (width 0.2) (layer "F.Cu") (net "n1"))
 (segment (start 25.1797 18.7844) (end 25.8553 19.46) (width 0.2) (layer "F.Cu") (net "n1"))
 (segment (start 25.1797 16.2422) (end 22.9375 14) (width 0.2) (layer "F.Cu") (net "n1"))
 (via (at 25.1797 18.7844) (size 0.6) (drill 0.3) (layers "F.Cu" "B.Cu") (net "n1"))
 (via (at 14.7973 49.0875) (size 0.6) (drill 0.3) (layers "F.Cu" "B.Cu") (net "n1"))
 (segment (start 25.1797 18.7844) (end 25.1797 38.7051) (width 0.2) (layer "B.Cu") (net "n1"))
 (segment (start 25.1797 38.7051) (end 14.7973 49.0875) (width 0.2) (layer "B.Cu") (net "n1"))
 (segment (start 39.7121 8.1517) (end 40 8.1517) (width 0.2) (layer "F.Cu") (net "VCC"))
 (segment (start 40.7291 24.0236) (end 40.7291 38.3491) (width 0.2) (layer "F.Cu") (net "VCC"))
 (segment (start 39.2162 21.4893) (end 39.2162 17.1234) (width 0.2) (layer "F.Cu") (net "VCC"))
 (segment (start 40 7) (end 40 8.1517) (width 0.2) (layer "F.Cu") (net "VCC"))
 (segment (start 38.3837 16.2909) (end 38.3837 9.4801) (width 0.2) (layer "F.Cu") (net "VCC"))
 (segment (start 38.7055 22) (end 39.2162 21.4893) (width 0.2) (layer "F.Cu") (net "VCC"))
 (segment (start 52.1695 23.8805) (end 40.8722 23.8805) (width 0.2) (layer "F.Cu") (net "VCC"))
 (segment (start 38.3837 9.4801) (end 39.7121 8.1517) (width 0.2) (layer "F.Cu") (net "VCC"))
 (segment (start 37.525 22) (end 38.7055 22) (width 0.2) (layer "F.Cu") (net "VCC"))
 (segment (start 54.05 22) (end 52.1695 23.8805) (width 0.2) (layer "F.Cu") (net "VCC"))
 (segment (start 38.7055 22) (end 40.7291 24.0236) (width 0.2) (layer "F.Cu") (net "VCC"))
 (segment (start 40.8722 23.8805) (end 40.7291 24.0236) (width 0.2) (layer "F.Cu") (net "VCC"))
 (segment (start 40.7291 38.3491) (end 42.475 40.095) (width 0.2) (layer "F.Cu") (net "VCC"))
 (segment (start 39.2162 17.1234) (end 38.3837 16.2909) (width 0.2) (layer "F.Cu") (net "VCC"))
 (segment (start 38.8245 26.2089) (end 35.0334 30) (width 0.2) (layer "F.Cu") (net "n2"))
 (segment (start 38.8245 25.4639) (end 38.8245 26.2089) (width 0.2) (layer "F.Cu") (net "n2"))
 (segment (start 22.9375 47.025) (end 22.9375 30) (width 0.2) (layer "F.Cu") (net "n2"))
 (segment (start 37.9006 24.54) (end 38.8245 25.4639) (width 0.2) (layer "F.Cu") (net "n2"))
 (segment (start 35.0334 30) (end 22.9375 30) (width 0.2) (layer "F.Cu") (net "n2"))
 (segment (start 37.525 24.54) (end 37.9006 24.54) (width 0.2) (layer "F.Cu") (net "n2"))
 (segment (start 25 49.0875) (end 22.9375 47.025) (width 0.2) (layer "F.Cu") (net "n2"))
 (segment (start 42.1427 50.0552) (end 41.9475 50.0552) (width 0.2) (layer "F.Cu") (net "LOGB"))
 (segment (start 24.9044 26.6456) (end 37.525 26.6456) (width 0.2) (layer "F.Cu") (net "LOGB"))
 (segment (start 43 50.9125) (end 42.1427 50.0552) (width 0.2) (layer "F.Cu") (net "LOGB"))
 (segment (start 37.525 26.6456) (end 37.525 25.81) (width 0.2) (layer "F.Cu") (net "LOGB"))
 (segment (start 21.0625 30.4875) (end 24.9044 26.6456) (width 0.2) (layer "F.Cu") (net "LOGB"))
 (segment (start 21.0625 30.95) (end 21.0625 30.4875) (width 0.2) (layer "F.Cu") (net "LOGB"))
 (via (at 41.9475 50.0552) (size 0.6) (drill 0.3) (layers "F.Cu" "B.Cu") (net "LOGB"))
 (via (at 37.525 26.6456) (size 0.6) (drill 0.3) (layers "F.Cu" "B.Cu") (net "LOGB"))
 (segment (start 41.9475 31.0681) (end 41.9475 50.0552) (width 0.2) (layer "B.Cu") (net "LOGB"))
 (segment (start 37.525 26.6456) (end 41.9475 31.0681) (width 0.2) (layer "B.Cu") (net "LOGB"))
 (segment (start 50.175 49.0875) (end 52 50.9125) (width 0.2) (layer "F.Cu") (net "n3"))
 (segment (start 42.475 24.54) (end 42.0741 24.54) (width 0.2) (layer "F.Cu") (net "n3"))
 (segment (start 42.5972 27.6225) (end 43.2518 27.6225) (width 0.2) (layer "F.Cu") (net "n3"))
 (segment (start 42.0741 24.54) (end 41.1574 25.4567) (width 0.2) (layer "F.Cu") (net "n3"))
 (segment (start 43 49.0875) (end 50.175 49.0875) (width 0.2) (layer "F.Cu") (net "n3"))
 (segment (start 41.1574 26.1827) (end 42.5972 27.6225) (width 0.2) (layer "F.Cu") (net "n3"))
 (segment (start 43 49.0875) (end 43 48.3203) (width 0.2) (layer "F.Cu") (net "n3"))
 (segment (start 41.1574 25.4567) (end 41.1574 26.1827) (width 0.2) (layer "F.Cu") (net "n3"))
 (segment (start 43 48.3203) (end 43.2518 48.0685) (width 0.2) (layer "F.Cu") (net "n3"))
 (segment (start 34 49.0875) (end 43 49.0875) (width 0.2) (layer "F.Cu") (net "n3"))
 (via (at 43.2518 48.0685) (size 0.6) (drill 0.3) (layers "F.Cu" "B.Cu") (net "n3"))
 (via (at 43.2518 27.6225) (size 0.6) (drill 0.3) (layers "F.Cu" "B.Cu") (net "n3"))
 (segment (start 43.2518 27.6225) (end 43.2518 48.0685) (width 0.2) (layer "B.Cu") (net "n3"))
 (segment (start 36.4967 42) (end 52.2261 42) (width 0.2) (layer "F.Cu") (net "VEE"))
 (segment (start 36.2427 42.9912) (end 36.2427 42.254) (width 0.2) (layer "F.Cu") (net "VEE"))
 (segment (start 42.1104 22) (end 39.6179 19.5075) (width 0.2) (layer "F.Cu") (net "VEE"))
 (segment (start 36.2427 42.254) (end 36.4967 42) (width 0.2) (layer "F.Cu") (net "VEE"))
 (segment (start 39.6179 19.5075) (end 39.6179 16.957) (width 0.2) (layer "F.Cu") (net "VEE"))
 (segment (start 38.8328 10.7072) (end 40 9.54) (width 0.2) (layer "F.Cu") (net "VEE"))
 (segment (start 52.2261 42) (end 53.4064 40.8197) (width 0.2) (layer "F.Cu") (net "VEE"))
 (segment (start 39.6179 16.957) (end 38.8328 16.1719) (width 0.2) (layer "F.Cu") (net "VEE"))
 (segment (start 53.4064 40.8197) (end 54.05 41.4633) (width 0.2) (layer "F.Cu") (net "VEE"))
 (segment (start 37.1565 43.905) (end 36.2427 42.9912) (width 0.2) (layer "F.Cu") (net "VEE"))
 (segment (start 37.525 43.905) (end 37.1565 43.905) (width 0.2) (layer "F.Cu") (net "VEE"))
 (segment (start 54.05 41.4633) (end 54.05 42) (width 0.2) (layer "F.Cu") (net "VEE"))
 (segment (start 42.475 22) (end 42.1104 22) (width 0.2) (layer "F.Cu") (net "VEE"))
 (segment (start 38.8328 16.1719) (end 38.8328 10.7072) (width 0.2) (layer "F.Cu") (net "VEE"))
 (via (at 53.4064 40.8197) (size 0.6) (drill 0.3) (layers "F.Cu" "B.Cu") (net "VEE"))
 (segment (start 53.4064 22.9464) (end 53.4064 40.8197) (width 0.2) (layer "B.Cu") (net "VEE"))
 (segment (start 40 9.54) (end 53.4064 22.9464) (width 0.2) (layer "B.Cu") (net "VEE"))
 (segment (start 72.2879 31.1517) (end 73.1668 32.0306) (width 0.2) (layer "F.Cu") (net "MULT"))
 (segment (start 42.475 18.19) (end 55.6355 18.19) (width 0.2) (layer "F.Cu") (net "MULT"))
 (segment (start 72 31.1517) (end 72.2879 31.1517) (width 0.2) (layer "F.Cu") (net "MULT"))
 (segment (start 73.1668 32.0306) (end 73.1668 36.9207) (width 0.2) (layer "F.Cu") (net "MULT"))
 (segment (start 72 30) (end 72 30.5758) (width 0.2) (layer "F.Cu") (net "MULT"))
 (segment (start 72 30.5758) (end 55.6355 30.5758) (width 0.2) (layer "F.Cu") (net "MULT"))
 (segment (start 72 30.5758) (end 72 31.1517) (width 0.2) (layer "F.Cu") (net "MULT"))
 (segment (start 73.1668 36.9207) (end 61 49.0875) (width 0.2) (layer "F.Cu") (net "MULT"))
 (via (at 55.6355 18.19) (size 0.6) (drill 0.3) (layers "F.Cu" "B.Cu") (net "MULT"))
 (via (at 55.6355 30.5758) (size 0.6) (drill 0.3) (layers "F.Cu" "B.Cu") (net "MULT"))
 (segment (start 55.6355 18.19) (end 55.6355 30.5758) (width 0.2) (layer "B.Cu") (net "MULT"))
 (segment (start 32.9988 42.9551) (end 32.9988 45.8256) (width 0.2) (layer "F.Cu") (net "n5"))
 (segment (start 26.0113 57.0988) (end 25 56.0875) (width 0.2) (layer "F.Cu") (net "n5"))
 (segment (start 38.8229 40.4735) (end 38.8229 39.7598) (width 0.2) (layer "F.Cu") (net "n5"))
 (segment (start 26.0113 58.425) (end 26.0113 57.9125) (width 0.2) (layer "F.Cu") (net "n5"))
 (segment (start 37.9314 41.365) (end 38.8229 40.4735) (width 0.2) (layer "F.Cu") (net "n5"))
 (segment (start 38.4959 39.4328) (end 36.5211 39.4328) (width 0.2) (layer "F.Cu") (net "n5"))
 (segment (start 25.6818 58.7545) (end 26.0113 58.425) (width 0.2) (layer "F.Cu") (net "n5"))
 (segment (start 16 56.0875) (end 18.667 58.7545) (width 0.2) (layer "F.Cu") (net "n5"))
 (segment (start 37.525 41.365) (end 37.9314 41.365) (width 0.2) (layer "F.Cu") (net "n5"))
 (segment (start 25 53.8244) (end 25 56.0875) (width 0.2) (layer "F.Cu") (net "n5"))
 (segment (start 32.9988 45.8256) (end 25 53.8244) (width 0.2) (layer "F.Cu") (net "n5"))
 (segment (start 26.0113 57.9125) (end 26.0113 57.0988) (width 0.2) (layer "F.Cu") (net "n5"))
 (segment (start 38.8229 39.7598) (end 38.4959 39.4328) (width 0.2) (layer "F.Cu") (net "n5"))
 (segment (start 26.0113 57.9125) (end 34 57.9125) (width 0.2) (layer "F.Cu") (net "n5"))
 (segment (start 36.5211 39.4328) (end 32.9988 42.9551) (width 0.2) (layer "F.Cu") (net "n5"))
 (segment (start 18.667 58.7545) (end 25.6818 58.7545) (width 0.2) (layer "F.Cu") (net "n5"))
 (segment (start 34.6008 46.7695) (end 32.9463 48.424) (width 0.2) (layer "F.Cu") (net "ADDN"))
 (segment (start 34.6008 42.6474) (end 34.6008 46.7695) (width 0.2) (layer "F.Cu") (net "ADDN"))
 (segment (start 35.825 57.9125) (end 34 56.0875) (width 0.2) (layer "F.Cu") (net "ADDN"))
 (segment (start 32.9463 48.424) (end 32.9463 55.0338) (width 0.2) (layer "F.Cu") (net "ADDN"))
 (segment (start 37.525 40.095) (end 37.1532 40.095) (width 0.2) (layer "F.Cu") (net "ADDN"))
 (segment (start 37.1532 40.095) (end 34.6008 42.6474) (width 0.2) (layer "F.Cu") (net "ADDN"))
 (segment (start 43 57.9125) (end 35.825 57.9125) (width 0.2) (layer "F.Cu") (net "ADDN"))
 (segment (start 32.9463 55.0338) (end 34 56.0875) (width 0.2) (layer "F.Cu") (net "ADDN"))
 (segment (start 52 57.9125) (end 49.763 55.6754) (width 0.2) (layer "F.Cu") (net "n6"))
 (segment (start 53.0036 51.8668) (end 52.3996 52.4708) (width 0.2) (layer "F.Cu") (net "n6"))
 (segment (start 43 56.0875) (end 49.3509 56.0875) (width 0.2) (layer "F.Cu") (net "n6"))
 (segment (start 52.3996 52.4708) (end 52.3996 53.0388) (width 0.2) (layer "F.Cu") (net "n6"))
 (segment (start 53.0036 48.5309) (end 53.0036 51.8668) (width 0.2) (layer "F.Cu") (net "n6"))
 (segment (start 52.1827 47.71) (end 53.0036 48.5309) (width 0.2) (layer "F.Cu") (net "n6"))
 (segment (start 51.3333 47.71) (end 52.1827 47.71) (width 0.2) (layer "F.Cu") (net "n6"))
 (segment (start 42.475 42.635) (end 46.2583 42.635) (width 0.2) (layer "F.Cu") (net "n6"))
 (segment (start 52.3996 53.0388) (end 49.763 55.6754) (width 0.2) (layer "F.Cu") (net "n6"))
 (segment (start 49.3509 56.0875) (end 49.763 55.6754) (width 0.2) (layer "F.Cu") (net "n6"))
 (segment (start 46.2583 42.635) (end 51.3333 47.71) (width 0.2) (layer "F.Cu") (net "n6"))
 (segment (start 54.9026 53.1849) (end 54.9026 40.1996) (width 0.2) (layer "F.Cu") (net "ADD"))
 (segment (start 54.9026 40.1996) (end 44.0609 40.1996) (width 0.2) (layer "F.Cu") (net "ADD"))
 (segment (start 42.8955 41.365) (end 42.475 41.365) (width 0.2) (layer "F.Cu") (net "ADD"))
 (segment (start 44.0609 40.1996) (end 42.8955 41.365) (width 0.2) (layer "F.Cu") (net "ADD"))
 (segment (start 52 56.0875) (end 54.9026 53.1849) (width 0.2) (layer "F.Cu") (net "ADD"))
 (segment (start 62.5622 32.54) (end 72 32.54) (width 0.2) (layer "F.Cu") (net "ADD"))
 (segment (start 54.9026 40.1996) (end 62.5622 32.54) (width 0.2) (layer "F.Cu") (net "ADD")))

